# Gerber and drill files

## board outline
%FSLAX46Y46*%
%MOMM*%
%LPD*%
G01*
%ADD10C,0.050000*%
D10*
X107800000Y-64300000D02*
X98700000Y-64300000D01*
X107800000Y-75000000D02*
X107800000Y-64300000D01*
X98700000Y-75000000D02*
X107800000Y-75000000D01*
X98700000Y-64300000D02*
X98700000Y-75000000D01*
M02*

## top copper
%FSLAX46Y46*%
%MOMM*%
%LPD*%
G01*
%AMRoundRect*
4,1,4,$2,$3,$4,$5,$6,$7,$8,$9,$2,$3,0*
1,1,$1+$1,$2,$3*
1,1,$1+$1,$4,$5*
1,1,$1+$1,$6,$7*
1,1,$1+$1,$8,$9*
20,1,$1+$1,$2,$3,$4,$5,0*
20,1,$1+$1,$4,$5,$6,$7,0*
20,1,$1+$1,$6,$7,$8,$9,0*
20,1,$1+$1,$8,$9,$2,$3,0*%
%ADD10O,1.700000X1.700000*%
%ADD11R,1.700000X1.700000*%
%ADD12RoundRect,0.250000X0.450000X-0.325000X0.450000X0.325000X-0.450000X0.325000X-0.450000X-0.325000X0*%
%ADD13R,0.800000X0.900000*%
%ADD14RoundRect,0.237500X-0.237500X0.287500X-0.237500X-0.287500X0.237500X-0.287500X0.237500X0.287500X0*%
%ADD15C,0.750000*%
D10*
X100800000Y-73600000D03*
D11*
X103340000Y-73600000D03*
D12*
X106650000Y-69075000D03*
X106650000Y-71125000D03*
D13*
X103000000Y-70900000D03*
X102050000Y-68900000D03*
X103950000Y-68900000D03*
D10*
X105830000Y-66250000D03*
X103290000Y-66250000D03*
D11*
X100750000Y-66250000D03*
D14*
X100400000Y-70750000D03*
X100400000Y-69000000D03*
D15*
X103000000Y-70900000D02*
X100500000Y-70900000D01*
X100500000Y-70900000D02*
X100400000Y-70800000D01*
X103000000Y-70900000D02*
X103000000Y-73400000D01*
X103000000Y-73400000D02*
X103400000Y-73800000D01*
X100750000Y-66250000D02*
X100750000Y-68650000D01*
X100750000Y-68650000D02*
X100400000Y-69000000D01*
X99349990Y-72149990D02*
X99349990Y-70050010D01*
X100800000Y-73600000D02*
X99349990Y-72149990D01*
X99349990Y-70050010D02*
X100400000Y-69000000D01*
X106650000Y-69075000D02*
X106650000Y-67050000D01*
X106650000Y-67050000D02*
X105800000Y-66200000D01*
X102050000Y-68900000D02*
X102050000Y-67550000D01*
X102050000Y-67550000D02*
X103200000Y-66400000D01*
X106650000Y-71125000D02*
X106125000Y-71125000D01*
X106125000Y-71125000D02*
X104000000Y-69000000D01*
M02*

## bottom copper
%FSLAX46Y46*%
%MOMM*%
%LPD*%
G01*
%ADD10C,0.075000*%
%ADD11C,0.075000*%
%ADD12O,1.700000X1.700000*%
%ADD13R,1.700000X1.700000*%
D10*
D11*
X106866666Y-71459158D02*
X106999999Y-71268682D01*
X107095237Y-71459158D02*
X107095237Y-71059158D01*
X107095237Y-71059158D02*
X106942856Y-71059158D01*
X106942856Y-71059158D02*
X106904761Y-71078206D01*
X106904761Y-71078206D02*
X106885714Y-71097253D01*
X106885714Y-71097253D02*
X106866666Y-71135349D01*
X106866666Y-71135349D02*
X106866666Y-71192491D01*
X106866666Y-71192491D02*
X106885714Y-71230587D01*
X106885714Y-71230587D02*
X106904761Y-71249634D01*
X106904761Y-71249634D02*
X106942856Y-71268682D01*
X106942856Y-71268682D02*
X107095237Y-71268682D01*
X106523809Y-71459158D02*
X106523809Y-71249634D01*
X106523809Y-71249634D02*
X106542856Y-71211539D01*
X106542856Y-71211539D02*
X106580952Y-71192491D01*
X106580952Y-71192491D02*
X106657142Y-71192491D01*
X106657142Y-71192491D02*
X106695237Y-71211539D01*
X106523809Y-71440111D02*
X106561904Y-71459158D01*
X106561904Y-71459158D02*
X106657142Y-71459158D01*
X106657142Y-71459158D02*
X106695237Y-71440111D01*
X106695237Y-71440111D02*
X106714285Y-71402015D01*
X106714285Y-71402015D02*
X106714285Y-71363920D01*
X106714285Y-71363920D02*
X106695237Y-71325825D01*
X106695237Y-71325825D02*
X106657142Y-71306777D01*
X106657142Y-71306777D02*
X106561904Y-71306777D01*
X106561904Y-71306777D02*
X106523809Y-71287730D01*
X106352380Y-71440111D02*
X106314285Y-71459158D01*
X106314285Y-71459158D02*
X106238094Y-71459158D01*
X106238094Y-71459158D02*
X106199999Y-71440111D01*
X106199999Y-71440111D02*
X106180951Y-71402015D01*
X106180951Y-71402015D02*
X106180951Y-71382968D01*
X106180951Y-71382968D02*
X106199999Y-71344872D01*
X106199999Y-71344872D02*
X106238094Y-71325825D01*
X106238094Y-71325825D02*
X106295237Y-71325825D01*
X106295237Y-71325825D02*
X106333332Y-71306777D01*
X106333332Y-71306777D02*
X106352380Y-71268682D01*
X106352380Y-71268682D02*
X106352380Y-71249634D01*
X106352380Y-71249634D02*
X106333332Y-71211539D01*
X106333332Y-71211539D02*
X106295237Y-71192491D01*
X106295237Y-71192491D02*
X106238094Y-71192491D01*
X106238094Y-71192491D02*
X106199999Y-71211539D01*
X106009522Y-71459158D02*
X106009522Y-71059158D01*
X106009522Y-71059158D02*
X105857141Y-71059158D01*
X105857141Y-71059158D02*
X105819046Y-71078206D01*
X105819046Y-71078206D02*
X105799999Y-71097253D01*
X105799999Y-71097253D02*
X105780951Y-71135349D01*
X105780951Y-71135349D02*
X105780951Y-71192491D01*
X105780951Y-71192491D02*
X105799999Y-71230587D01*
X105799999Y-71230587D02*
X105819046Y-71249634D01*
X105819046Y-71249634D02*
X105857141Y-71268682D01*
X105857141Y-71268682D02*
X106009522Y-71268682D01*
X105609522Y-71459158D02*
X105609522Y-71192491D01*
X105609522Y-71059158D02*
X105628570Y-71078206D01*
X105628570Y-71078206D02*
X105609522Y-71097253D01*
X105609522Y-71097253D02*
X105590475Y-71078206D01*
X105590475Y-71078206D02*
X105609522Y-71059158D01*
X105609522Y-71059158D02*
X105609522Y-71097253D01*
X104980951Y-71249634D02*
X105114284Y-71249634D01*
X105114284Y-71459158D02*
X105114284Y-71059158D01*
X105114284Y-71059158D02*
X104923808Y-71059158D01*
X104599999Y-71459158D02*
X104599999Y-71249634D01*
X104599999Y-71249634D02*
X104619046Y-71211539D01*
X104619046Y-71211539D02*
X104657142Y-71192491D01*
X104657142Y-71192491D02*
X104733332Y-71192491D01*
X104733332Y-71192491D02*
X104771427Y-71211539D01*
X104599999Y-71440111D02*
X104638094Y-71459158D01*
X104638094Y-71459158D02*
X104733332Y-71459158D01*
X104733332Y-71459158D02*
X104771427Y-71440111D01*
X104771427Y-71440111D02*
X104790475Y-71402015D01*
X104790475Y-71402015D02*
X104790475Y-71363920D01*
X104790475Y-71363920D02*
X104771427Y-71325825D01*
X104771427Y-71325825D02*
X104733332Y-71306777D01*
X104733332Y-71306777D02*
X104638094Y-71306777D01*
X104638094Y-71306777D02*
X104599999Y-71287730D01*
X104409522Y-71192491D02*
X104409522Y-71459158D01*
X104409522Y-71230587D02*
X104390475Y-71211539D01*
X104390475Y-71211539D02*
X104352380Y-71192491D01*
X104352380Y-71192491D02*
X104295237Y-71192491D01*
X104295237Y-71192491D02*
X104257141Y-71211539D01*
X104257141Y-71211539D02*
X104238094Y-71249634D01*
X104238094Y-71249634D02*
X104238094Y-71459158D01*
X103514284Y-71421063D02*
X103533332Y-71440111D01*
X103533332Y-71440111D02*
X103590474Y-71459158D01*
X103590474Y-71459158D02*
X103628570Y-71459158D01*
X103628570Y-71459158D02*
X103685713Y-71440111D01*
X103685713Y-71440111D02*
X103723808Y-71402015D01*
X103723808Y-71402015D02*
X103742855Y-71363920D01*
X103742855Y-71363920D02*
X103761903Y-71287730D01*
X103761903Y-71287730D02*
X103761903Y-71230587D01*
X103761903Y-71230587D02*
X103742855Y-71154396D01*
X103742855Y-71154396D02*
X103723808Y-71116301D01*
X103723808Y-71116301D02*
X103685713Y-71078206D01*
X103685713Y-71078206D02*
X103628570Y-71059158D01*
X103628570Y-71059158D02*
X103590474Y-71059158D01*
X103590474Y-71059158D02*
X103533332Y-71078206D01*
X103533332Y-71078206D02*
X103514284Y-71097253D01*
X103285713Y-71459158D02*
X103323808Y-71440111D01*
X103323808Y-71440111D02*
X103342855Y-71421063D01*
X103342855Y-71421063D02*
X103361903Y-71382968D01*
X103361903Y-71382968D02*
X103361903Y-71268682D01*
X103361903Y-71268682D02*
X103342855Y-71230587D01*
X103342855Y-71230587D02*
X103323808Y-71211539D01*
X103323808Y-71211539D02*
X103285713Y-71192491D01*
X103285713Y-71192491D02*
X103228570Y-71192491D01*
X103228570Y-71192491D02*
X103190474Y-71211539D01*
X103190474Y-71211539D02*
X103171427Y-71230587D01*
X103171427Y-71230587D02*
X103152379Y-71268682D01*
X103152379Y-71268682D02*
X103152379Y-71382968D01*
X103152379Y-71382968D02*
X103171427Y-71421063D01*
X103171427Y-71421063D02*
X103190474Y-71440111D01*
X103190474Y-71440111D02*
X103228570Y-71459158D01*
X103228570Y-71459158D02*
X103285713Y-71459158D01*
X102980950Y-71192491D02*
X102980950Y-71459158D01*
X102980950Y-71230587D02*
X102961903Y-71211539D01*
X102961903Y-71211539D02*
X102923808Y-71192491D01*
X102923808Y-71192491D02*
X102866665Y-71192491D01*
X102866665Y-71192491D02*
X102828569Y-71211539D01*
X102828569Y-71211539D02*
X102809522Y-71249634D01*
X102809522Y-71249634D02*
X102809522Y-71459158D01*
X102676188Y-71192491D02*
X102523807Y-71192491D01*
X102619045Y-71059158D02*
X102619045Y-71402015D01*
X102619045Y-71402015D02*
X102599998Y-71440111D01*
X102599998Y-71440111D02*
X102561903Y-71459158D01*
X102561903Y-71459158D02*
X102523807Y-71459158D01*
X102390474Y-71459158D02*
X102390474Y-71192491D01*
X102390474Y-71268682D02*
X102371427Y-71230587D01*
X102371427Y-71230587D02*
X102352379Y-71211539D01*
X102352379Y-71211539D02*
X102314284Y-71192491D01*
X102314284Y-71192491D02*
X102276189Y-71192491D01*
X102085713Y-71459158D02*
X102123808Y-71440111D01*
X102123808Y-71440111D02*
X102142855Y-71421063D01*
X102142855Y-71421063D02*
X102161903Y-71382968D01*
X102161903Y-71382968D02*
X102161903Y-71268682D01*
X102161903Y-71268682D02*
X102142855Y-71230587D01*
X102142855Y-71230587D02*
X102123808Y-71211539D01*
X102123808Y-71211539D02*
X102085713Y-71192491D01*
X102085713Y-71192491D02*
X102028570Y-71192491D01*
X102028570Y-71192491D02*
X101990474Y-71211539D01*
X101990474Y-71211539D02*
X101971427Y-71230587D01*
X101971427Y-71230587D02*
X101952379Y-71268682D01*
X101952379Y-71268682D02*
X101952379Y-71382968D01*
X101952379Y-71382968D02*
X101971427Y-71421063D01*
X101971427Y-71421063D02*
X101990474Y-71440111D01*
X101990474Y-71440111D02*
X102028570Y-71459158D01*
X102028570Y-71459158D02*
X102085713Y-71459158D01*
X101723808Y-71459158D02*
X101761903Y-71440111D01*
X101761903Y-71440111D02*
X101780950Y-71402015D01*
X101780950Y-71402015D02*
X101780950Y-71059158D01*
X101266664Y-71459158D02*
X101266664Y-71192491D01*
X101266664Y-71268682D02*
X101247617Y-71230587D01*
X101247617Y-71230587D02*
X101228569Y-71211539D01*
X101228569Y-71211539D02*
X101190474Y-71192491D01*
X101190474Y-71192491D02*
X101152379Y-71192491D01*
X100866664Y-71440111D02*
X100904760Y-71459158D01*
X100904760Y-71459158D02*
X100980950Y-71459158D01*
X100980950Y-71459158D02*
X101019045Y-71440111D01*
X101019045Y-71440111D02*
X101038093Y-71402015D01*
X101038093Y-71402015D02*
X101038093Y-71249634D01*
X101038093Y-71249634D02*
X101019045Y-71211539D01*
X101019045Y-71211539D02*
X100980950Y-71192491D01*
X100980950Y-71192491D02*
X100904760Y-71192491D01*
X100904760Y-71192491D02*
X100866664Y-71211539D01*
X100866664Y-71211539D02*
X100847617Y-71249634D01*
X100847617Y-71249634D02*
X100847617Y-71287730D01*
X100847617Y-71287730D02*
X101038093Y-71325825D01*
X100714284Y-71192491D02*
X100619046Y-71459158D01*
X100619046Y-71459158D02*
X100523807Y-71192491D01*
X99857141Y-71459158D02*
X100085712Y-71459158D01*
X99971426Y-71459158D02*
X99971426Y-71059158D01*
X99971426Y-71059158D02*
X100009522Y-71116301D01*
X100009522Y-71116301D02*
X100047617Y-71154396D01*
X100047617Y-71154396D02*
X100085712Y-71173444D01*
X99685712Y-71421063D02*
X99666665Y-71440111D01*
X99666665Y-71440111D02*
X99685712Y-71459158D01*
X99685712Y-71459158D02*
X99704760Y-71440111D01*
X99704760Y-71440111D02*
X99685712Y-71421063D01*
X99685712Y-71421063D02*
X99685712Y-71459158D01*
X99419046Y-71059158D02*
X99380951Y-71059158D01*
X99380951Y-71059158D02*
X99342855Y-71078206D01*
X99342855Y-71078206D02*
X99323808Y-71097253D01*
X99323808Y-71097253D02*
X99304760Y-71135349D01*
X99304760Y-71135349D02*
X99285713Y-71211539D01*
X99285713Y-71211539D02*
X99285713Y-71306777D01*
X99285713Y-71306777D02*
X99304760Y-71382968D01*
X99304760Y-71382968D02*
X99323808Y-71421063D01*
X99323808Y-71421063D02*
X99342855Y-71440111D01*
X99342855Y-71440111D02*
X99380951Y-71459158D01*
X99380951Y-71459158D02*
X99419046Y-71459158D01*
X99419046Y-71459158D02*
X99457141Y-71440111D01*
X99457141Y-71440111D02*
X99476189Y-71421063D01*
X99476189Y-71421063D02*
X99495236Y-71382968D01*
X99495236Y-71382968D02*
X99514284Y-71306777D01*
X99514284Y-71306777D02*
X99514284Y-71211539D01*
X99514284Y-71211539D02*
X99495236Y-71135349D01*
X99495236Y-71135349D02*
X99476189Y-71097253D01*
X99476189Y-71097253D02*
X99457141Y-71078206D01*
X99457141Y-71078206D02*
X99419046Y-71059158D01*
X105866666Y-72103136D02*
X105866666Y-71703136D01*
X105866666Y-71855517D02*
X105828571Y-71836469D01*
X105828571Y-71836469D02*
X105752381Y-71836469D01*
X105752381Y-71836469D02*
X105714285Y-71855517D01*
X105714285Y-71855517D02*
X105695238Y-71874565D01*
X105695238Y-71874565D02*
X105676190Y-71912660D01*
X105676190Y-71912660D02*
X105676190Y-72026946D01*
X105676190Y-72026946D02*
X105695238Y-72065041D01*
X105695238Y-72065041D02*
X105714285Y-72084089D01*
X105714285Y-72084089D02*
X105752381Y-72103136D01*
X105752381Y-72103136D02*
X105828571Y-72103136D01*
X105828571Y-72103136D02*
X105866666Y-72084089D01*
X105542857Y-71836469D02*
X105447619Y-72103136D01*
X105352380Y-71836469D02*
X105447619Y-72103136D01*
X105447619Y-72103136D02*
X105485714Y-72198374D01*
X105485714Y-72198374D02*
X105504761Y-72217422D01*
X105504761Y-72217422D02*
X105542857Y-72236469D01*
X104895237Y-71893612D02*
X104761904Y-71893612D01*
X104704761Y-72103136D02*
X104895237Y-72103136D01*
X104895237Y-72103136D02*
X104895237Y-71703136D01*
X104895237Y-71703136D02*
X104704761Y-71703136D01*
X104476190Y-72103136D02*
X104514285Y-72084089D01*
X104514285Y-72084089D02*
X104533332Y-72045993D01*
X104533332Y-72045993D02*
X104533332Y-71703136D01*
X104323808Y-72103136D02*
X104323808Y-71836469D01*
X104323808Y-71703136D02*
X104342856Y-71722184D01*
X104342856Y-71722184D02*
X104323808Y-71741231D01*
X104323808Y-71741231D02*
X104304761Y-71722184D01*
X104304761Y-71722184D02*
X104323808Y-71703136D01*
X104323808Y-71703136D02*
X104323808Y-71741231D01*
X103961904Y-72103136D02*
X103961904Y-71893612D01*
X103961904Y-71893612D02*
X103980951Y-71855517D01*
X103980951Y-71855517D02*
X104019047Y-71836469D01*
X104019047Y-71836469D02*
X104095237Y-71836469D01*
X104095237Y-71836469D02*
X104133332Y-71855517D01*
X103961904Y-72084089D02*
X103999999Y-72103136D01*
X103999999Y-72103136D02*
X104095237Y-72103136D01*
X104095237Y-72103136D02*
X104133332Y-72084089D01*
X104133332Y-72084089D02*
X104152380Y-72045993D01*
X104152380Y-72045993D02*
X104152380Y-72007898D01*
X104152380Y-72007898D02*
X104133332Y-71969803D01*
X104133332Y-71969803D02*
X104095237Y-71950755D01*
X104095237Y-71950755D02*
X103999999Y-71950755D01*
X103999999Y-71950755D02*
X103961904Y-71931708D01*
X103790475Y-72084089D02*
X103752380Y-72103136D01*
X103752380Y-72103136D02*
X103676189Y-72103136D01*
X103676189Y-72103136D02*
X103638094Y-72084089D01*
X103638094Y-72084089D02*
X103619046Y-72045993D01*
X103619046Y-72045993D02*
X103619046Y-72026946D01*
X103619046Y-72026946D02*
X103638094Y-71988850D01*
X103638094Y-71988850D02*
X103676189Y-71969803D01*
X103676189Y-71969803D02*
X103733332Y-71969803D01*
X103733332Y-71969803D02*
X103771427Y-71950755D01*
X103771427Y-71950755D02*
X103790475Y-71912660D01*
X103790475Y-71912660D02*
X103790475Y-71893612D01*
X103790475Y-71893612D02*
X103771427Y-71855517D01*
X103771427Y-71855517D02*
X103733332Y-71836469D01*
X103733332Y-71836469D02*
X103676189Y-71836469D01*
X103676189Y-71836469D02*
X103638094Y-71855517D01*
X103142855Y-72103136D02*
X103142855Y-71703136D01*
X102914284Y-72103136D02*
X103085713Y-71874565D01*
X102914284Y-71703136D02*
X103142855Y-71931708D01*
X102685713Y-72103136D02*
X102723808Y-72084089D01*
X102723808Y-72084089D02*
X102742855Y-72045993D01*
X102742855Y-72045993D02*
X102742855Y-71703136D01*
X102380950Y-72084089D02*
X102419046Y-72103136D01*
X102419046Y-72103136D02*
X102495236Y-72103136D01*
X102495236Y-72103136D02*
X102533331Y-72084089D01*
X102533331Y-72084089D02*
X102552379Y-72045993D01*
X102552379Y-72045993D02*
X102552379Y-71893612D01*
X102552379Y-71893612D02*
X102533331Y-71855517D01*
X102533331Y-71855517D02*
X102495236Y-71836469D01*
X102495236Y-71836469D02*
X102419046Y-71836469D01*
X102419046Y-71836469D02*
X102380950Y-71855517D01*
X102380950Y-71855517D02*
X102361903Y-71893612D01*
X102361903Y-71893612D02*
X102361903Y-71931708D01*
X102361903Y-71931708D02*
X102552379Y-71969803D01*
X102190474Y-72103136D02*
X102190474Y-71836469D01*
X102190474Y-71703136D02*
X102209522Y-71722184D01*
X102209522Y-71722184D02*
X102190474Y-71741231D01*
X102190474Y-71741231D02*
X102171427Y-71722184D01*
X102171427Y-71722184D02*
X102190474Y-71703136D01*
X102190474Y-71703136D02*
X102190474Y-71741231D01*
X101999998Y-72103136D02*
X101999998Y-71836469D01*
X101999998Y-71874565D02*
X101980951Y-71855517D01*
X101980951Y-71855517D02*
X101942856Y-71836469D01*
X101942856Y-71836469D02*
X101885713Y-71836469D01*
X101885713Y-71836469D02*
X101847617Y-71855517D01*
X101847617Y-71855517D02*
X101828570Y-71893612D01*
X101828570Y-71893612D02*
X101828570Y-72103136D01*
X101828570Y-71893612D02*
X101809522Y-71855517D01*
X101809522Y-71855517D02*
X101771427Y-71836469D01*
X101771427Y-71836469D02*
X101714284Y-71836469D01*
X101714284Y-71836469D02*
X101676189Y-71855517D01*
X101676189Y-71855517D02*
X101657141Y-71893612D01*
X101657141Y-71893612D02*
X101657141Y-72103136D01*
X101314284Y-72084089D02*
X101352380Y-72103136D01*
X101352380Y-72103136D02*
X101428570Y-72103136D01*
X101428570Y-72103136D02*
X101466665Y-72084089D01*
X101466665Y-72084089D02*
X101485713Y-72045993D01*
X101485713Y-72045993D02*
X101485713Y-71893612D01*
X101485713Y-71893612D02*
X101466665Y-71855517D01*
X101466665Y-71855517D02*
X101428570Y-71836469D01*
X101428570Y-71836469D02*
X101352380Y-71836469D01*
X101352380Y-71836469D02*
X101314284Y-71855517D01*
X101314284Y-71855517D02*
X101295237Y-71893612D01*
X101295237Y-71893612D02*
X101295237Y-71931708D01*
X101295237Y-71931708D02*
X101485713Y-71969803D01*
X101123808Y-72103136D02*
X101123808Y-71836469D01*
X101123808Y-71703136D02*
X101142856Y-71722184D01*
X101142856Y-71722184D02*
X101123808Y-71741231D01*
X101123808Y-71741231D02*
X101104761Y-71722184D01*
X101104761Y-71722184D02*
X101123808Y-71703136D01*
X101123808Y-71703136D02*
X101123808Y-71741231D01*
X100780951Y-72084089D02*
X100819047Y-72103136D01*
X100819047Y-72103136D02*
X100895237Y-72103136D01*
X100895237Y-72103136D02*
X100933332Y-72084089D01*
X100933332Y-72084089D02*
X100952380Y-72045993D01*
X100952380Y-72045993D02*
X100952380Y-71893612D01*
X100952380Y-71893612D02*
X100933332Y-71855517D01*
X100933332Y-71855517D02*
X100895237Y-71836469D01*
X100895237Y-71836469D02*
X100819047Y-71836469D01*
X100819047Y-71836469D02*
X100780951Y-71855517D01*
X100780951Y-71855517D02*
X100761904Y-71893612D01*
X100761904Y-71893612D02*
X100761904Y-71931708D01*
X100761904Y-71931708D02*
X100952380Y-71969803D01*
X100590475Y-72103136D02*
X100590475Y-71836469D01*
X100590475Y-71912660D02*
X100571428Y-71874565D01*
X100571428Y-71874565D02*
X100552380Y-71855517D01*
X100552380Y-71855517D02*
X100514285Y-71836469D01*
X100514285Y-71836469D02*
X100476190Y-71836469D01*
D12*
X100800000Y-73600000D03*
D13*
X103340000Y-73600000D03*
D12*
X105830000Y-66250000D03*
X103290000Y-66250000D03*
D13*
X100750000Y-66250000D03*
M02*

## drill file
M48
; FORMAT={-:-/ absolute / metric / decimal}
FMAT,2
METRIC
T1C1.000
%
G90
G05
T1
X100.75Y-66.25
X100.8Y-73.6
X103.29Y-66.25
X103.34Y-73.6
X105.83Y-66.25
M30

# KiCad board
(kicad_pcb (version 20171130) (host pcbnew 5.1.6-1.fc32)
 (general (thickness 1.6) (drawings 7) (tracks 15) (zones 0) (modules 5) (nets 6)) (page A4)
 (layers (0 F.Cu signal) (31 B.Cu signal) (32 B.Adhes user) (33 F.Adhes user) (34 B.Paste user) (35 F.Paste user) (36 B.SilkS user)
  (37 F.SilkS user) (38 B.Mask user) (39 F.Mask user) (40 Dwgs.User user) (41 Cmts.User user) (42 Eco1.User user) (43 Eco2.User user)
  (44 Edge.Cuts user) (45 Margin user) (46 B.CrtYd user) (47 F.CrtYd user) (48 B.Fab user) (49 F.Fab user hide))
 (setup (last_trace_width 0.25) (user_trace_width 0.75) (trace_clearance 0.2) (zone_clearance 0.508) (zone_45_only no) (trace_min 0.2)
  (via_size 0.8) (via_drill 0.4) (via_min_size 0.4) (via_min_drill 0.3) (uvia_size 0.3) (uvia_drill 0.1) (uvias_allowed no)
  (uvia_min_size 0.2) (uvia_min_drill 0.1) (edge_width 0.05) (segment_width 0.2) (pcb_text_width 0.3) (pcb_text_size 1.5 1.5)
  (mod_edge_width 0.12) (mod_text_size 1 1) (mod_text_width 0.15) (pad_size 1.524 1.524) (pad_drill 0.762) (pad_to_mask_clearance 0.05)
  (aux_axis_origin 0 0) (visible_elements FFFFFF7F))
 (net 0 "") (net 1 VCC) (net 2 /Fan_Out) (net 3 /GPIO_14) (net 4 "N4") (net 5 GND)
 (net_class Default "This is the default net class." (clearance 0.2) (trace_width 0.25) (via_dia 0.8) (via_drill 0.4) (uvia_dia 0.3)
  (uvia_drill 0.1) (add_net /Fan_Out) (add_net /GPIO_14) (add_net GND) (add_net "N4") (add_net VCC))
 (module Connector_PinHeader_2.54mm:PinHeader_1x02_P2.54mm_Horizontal (layer F.Cu) (at 103.34 73.6 270)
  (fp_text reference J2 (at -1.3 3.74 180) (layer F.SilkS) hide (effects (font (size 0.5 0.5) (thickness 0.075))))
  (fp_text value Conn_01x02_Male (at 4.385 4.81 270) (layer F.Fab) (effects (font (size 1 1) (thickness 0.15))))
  (pad 2 thru_hole oval (at 0 2.54 270) (size 1.7 1.7) (drill 1) (layers *.Cu *.Mask) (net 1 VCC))
  (pad 1 thru_hole rect (at 0 0 270) (size 1.7 1.7) (drill 1) (layers *.Cu *.Mask) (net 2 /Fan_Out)))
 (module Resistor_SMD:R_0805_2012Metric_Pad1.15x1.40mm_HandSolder (layer F.Cu) (at 106.65 70.1 90)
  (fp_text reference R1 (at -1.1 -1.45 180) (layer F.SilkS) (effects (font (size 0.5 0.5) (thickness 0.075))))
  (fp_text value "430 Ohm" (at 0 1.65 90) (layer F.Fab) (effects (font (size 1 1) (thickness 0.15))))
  (pad 2 smd roundrect (at 1.025 0 90) (size 1.15 1.4) (layers F.Cu F.Paste F.Mask) (roundrect_rratio 0.217391) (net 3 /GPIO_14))
  (pad 1 smd roundrect (at -1.025 0 90) (size 1.15 1.4) (layers F.Cu F.Paste F.Mask) (roundrect_rratio 0.217391) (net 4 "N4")))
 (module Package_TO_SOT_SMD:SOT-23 (layer F.Cu) (at 103 69.9 270)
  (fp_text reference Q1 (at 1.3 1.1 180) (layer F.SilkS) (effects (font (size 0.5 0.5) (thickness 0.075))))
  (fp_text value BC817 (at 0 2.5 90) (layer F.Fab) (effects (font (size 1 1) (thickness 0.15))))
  (pad 3 smd rect (at 1 0 270) (size 0.9 0.8) (layers F.Cu F.Paste F.Mask) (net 2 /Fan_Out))
  (pad 2 smd rect (at -1 0.95 270) (size 0.9 0.8) (layers F.Cu F.Paste F.Mask) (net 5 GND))
  (pad 1 smd rect (at -1 -0.95 270) (size 0.9 0.8) (layers F.Cu F.Paste F.Mask) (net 4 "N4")))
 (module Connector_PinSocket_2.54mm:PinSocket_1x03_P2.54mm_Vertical (layer B.Cu) (at 100.75 66.25 270)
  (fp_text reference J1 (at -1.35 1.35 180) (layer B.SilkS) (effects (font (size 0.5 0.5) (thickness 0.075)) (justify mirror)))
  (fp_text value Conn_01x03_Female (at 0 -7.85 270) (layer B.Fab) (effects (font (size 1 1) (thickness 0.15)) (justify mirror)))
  (pad 3 thru_hole oval (at 0 -5.08 270) (size 1.7 1.7) (drill 1) (layers *.Cu *.Mask) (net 3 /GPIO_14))
  (pad 2 thru_hole oval (at 0 -2.54 270) (size 1.7 1.7) (drill 1) (layers *.Cu *.Mask) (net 5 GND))
  (pad 1 thru_hole rect (at 0 0 270) (size 1.7 1.7) (drill 1) (layers *.Cu *.Mask) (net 1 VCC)))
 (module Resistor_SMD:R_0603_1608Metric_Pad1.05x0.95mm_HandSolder (layer F.Cu) (at 100.4 69.875 270)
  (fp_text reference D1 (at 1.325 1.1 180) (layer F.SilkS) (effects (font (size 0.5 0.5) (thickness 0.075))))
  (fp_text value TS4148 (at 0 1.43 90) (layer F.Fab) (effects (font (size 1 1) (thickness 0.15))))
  (pad 2 smd roundrect (at 0.875 0 270) (size 1.05 0.95) (layers F.Cu F.Paste F.Mask) (roundrect_rratio 0.25) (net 2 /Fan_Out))
  (pad 1 smd roundrect (at -0.875 0 270) (size 1.05 0.95) (layers F.Cu F.Paste F.Mask) (roundrect_rratio 0.25) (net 1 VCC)))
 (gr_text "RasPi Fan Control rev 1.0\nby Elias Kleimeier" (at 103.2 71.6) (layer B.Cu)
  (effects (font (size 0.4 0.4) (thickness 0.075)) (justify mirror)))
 (gr_line (start 107.8 64.3) (end 98.7 64.3) (layer Edge.Cuts) (width 0.05))
 (gr_line (start 107.8 75) (end 107.8 64.3) (layer Edge.Cuts) (width 0.05))
 (gr_line (start 98.7 75) (end 107.8 75) (layer Edge.Cuts) (width 0.05))
 (gr_line (start 98.7 64.3) (end 98.7 75) (layer Edge.Cuts) (width 0.05))
 (segment (start 103 70.9) (end 100.5 70.9) (width 0.75) (layer F.Cu) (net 2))
 (segment (start 100.5 70.9) (end 100.4 70.8) (width 0.75) (layer F.Cu) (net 2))
 (segment (start 103 70.9) (end 103 73.4) (width 0.75) (layer F.Cu) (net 2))
 (segment (start 103 73.4) (end 103.4 73.8) (width 0.75) (layer F.Cu) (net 2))
 (segment (start 100.75 66.25) (end 100.75 68.65) (width 0.75) (layer F.Cu) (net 1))
 (segment (start 100.75 68.65) (end 100.4 69) (width 0.75) (layer F.Cu) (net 1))
 (segment (start 99.34999 72.14999) (end 99.34999 70.05001) (width 0.75) (layer F.Cu) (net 1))
 (segment (start 100.8 73.6) (end 99.34999 72.14999) (width 0.75) (layer F.Cu) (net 1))
 (segment (start 99.34999 70.05001) (end 100.4 69) (width 0.75) (layer F.Cu) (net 1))
 (segment (start 106.65 69.075) (end 106.65 67.05) (width 0.75) (layer F.Cu) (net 3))
 (segment (start 106.65 67.05) (end 105.8 66.2) (width 0.75) (layer F.Cu) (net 3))
 (segment (start 102.05 68.9) (end 102.05 67.55) (width 0.75) (layer F.Cu) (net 5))
 (segment (start 102.05 67.55) (end 103.2 66.4) (width 0.75) (layer F.Cu) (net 5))
 (segment (start 106.65 71.125) (end 106.125 71.125) (width 0.75) (layer F.Cu) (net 4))
 (segment (start 106.125 71.125) (end 104 69) (width 0.75) (layer F.Cu) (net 4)))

